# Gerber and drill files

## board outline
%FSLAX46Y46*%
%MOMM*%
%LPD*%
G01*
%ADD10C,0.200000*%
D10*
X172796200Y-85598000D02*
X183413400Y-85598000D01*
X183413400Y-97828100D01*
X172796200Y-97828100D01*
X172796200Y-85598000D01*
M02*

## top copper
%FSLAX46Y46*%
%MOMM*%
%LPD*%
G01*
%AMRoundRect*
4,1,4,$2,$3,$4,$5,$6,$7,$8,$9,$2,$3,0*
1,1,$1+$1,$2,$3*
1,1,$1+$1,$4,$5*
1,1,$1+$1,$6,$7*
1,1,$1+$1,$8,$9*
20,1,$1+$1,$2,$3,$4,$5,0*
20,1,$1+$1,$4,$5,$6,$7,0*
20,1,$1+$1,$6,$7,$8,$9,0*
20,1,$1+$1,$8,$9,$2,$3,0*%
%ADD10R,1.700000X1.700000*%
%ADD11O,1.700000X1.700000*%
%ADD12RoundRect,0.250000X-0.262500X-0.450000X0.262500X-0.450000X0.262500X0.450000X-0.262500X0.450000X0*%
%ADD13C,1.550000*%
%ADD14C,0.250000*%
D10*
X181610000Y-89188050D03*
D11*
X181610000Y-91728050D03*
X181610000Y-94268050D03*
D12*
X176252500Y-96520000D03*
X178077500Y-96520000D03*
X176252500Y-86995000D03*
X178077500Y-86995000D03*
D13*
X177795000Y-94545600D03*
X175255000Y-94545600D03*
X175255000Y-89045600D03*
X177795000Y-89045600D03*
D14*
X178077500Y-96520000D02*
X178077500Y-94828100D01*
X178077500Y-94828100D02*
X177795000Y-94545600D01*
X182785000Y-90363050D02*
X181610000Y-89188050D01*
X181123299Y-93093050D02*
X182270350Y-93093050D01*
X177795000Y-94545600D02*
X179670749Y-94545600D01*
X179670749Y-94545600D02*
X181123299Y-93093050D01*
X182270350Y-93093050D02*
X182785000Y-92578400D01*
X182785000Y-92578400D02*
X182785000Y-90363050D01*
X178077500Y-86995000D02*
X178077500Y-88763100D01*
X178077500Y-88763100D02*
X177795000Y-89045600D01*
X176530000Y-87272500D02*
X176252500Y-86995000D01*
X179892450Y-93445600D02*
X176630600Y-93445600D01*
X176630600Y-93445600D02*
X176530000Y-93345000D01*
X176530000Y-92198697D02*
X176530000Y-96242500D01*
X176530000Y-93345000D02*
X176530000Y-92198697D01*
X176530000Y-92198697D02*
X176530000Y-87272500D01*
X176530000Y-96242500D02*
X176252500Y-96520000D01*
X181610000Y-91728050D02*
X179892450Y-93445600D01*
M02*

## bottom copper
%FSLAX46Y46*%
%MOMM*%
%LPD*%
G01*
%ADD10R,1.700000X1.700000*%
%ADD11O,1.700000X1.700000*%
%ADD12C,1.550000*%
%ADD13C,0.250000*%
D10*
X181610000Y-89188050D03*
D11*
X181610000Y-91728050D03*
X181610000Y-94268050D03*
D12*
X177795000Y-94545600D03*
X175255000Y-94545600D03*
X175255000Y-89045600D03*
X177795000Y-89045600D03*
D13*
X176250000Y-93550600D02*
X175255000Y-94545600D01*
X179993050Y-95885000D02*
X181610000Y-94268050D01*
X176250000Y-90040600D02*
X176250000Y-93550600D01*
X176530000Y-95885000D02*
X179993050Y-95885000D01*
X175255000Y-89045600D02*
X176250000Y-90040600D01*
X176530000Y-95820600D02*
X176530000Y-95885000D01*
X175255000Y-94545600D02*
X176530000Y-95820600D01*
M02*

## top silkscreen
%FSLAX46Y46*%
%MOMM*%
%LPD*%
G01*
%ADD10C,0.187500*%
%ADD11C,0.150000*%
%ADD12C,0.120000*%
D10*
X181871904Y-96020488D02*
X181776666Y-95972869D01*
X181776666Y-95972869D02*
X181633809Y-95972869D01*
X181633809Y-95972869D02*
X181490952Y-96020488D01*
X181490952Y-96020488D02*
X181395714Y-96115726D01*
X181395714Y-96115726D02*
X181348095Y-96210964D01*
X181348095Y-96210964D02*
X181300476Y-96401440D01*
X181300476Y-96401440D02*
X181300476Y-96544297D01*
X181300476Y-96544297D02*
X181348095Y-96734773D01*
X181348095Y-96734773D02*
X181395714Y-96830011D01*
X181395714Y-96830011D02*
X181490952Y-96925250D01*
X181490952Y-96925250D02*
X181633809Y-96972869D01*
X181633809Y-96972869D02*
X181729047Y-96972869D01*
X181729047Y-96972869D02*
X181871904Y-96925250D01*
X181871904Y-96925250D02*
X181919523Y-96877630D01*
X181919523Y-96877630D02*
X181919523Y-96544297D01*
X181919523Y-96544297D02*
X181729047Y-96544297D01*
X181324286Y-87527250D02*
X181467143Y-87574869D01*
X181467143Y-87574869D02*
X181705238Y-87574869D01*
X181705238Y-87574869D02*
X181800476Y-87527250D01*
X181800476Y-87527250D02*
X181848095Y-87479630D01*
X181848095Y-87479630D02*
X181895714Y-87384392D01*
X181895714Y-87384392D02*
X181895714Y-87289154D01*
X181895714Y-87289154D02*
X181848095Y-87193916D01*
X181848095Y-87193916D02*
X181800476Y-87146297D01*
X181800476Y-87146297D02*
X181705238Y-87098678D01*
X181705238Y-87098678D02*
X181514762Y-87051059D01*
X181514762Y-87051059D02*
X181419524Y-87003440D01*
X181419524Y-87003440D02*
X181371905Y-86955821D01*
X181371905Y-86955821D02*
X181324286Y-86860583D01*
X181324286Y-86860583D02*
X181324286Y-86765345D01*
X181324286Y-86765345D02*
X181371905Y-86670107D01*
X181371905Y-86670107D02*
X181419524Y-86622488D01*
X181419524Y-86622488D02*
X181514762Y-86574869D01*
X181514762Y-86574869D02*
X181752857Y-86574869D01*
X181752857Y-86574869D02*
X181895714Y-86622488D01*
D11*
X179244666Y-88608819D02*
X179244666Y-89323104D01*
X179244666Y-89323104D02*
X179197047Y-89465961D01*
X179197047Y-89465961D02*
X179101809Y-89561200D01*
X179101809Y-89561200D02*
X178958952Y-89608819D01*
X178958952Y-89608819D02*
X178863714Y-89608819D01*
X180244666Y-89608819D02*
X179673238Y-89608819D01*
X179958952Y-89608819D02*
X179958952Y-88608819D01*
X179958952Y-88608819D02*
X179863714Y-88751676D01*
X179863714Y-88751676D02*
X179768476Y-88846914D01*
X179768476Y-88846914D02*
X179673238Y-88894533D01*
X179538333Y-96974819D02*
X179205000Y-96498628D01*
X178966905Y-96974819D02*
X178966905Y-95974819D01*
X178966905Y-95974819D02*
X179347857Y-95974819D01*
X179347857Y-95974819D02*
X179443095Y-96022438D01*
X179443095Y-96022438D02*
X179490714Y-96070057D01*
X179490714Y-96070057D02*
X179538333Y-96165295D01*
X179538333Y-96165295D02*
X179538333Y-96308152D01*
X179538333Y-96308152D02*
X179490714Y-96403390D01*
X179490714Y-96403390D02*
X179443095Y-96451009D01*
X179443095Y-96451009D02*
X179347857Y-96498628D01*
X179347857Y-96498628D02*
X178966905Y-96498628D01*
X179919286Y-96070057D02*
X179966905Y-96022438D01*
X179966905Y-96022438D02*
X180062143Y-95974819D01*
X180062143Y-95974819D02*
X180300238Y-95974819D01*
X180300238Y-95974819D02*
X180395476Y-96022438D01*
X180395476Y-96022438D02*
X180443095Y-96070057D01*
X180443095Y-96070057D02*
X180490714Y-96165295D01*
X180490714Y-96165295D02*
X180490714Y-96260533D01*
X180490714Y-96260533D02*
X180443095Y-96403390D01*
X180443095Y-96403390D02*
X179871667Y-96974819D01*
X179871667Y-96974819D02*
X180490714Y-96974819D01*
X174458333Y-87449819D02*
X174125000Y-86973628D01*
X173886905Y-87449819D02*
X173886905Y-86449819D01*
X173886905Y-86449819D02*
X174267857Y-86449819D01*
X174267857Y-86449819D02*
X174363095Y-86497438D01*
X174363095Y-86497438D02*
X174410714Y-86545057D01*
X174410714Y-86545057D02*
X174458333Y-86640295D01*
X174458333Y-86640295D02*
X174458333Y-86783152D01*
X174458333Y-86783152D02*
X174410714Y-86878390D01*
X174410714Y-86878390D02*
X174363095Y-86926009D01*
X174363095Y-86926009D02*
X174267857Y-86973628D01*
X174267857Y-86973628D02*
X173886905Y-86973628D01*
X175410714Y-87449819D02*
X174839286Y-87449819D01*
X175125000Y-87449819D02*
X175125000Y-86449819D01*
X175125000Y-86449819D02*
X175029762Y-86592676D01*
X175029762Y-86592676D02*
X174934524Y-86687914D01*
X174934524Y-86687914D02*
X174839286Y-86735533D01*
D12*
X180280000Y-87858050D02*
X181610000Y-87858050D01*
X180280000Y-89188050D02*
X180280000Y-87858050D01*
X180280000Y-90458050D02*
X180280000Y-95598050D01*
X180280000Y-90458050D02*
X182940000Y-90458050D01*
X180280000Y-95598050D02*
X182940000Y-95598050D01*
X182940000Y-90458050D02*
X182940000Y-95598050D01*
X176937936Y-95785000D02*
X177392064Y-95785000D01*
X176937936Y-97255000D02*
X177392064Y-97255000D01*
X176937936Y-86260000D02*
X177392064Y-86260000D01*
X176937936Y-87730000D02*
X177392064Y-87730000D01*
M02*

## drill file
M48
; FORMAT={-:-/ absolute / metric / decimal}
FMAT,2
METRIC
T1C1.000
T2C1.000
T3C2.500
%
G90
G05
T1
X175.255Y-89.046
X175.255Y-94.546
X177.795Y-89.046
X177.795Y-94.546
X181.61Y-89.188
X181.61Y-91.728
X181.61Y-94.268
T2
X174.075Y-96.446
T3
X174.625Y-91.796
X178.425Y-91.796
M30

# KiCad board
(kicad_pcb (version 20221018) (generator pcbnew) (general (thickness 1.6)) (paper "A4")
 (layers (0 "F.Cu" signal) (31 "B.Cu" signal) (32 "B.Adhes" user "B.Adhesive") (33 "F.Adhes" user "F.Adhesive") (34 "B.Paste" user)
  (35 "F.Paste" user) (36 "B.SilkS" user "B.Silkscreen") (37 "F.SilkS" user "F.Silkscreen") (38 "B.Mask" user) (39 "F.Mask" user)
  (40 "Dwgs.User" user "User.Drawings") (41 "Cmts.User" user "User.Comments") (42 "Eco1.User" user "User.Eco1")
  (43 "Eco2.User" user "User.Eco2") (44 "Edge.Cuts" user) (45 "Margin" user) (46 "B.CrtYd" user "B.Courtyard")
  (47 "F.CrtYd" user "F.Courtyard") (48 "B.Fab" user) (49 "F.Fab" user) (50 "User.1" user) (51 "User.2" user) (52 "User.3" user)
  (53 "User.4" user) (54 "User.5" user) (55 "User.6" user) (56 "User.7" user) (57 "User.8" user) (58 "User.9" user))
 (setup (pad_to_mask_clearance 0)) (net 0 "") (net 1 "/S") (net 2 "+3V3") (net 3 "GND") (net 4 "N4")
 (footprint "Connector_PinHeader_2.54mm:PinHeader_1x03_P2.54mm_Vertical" (layer "F.Cu") (at 181.61 89.18805)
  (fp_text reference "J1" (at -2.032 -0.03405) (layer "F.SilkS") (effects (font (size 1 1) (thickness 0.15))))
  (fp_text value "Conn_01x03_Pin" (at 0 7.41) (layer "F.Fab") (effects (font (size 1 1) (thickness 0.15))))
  (fp_line (start -1.33 -1.33) (end 0 -1.33) (stroke (width 0.12) (type solid)) (layer "F.SilkS"))
  (fp_line (start -1.33 0) (end -1.33 -1.33) (stroke (width 0.12) (type solid)) (layer "F.SilkS"))
  (fp_line (start -1.33 1.27) (end -1.33 6.41) (stroke (width 0.12) (type solid)) (layer "F.SilkS"))
  (fp_line (start -1.33 1.27) (end 1.33 1.27) (stroke (width 0.12) (type solid)) (layer "F.SilkS"))
  (fp_line (start -1.33 6.41) (end 1.33 6.41) (stroke (width 0.12) (type solid)) (layer "F.SilkS"))
  (fp_line (start 1.33 1.27) (end 1.33 6.41) (stroke (width 0.12) (type solid)) (layer "F.SilkS"))
  (pad "1" thru_hole rect (at 0 0) (size 1.7 1.7) (drill 1) (layers "*.Cu" "*.Mask") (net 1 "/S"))
  (pad "2" thru_hole oval (at 0 2.54) (size 1.7 1.7) (drill 1) (layers "*.Cu" "*.Mask") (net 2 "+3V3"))
  (pad "3" thru_hole oval (at 0 5.08) (size 1.7 1.7) (drill 1) (layers "*.Cu" "*.Mask") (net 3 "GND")))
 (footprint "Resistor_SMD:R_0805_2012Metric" (layer "F.Cu") (at 177.165 96.52)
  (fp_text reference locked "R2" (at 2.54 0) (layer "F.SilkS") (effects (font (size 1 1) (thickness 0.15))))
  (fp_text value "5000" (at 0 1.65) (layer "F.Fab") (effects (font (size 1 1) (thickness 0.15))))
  (fp_line (start -0.227064 -0.735) (end 0.227064 -0.735) (stroke (width 0.12) (type solid)) (layer "F.SilkS"))
  (fp_line (start -0.227064 0.735) (end 0.227064 0.735) (stroke (width 0.12) (type solid)) (layer "F.SilkS"))
  (pad "1" smd roundrect (at -0.9125 0) (size 1.025 1.4) (layers "F.Cu" "F.Paste" "F.Mask") (roundrect_rratio 0.243902439) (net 2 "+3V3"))
  (pad "2" smd roundrect (at 0.9125 0) (size 1.025 1.4) (layers "F.Cu" "F.Paste" "F.Mask") (roundrect_rratio 0.243902439) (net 1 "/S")))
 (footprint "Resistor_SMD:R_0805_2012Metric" (layer "F.Cu") (at 177.165 86.995)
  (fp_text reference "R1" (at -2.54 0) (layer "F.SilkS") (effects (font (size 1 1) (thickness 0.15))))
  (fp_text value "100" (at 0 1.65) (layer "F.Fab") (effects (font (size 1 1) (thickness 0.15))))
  (fp_line (start -0.227064 -0.735) (end 0.227064 -0.735) (stroke (width 0.12) (type solid)) (layer "F.SilkS"))
  (fp_line (start -0.227064 0.735) (end 0.227064 0.735) (stroke (width 0.12) (type solid)) (layer "F.SilkS"))
  (pad "1" smd roundrect (at -0.9125 0) (size 1.025 1.4) (layers "F.Cu" "F.Paste" "F.Mask") (roundrect_rratio 0.243902439) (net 2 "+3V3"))
  (pad "2" smd roundrect (at 0.9125 0) (size 1.025 1.4) (layers "F.Cu" "F.Paste" "F.Mask") (roundrect_rratio 0.243902439) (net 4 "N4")))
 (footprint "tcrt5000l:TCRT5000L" (layer "B.Cu") (at 176.525 91.7956 90)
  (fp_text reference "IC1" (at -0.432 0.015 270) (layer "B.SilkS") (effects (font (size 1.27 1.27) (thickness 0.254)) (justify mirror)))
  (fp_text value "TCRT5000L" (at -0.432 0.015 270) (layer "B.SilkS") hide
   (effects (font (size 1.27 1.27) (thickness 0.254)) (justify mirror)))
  (pad "" np_thru_hole circle (at -4.65 -2.45 90) (size 0.001 0.001) (drill 1) (layers "*.Cu" "*.Mask"))
  (pad "" np_thru_hole circle (at 0 -1.9 90) (size 0.001 0.001) (drill 2.5) (layers "*.Cu" "*.Mask"))
  (pad "" np_thru_hole circle (at 0 1.9 90) (size 0.001 0.001) (drill 2.5) (layers "*.Cu" "*.Mask"))
  (pad "1" thru_hole circle (at -2.75 1.27 90) (size 1.55 1.55) (drill 1) (layers "*.Cu" "*.Mask") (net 1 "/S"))
  (pad "2" thru_hole circle (at -2.75 -1.27 90) (size 1.55 1.55) (drill 1) (layers "*.Cu" "*.Mask") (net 3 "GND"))
  (pad "3" thru_hole circle (at 2.75 -1.27 90) (size 1.55 1.55) (drill 1) (layers "*.Cu" "*.Mask") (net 3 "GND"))
  (pad "4" thru_hole circle (at 2.75 1.27 90) (size 1.55 1.55) (drill 1) (layers "*.Cu" "*.Mask") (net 4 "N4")))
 (gr_rect (start 172.7962 85.598) (end 183.4134 97.8281) (stroke (width 0.2) (type solid)) (fill none) (layer "Edge.Cuts"))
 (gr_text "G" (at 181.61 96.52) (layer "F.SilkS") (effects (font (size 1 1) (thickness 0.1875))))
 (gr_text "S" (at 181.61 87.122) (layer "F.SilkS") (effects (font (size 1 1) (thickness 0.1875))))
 (segment (start 178.0775 96.52) (end 178.0775 94.8281) (width 0.25) (layer "F.Cu") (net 1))
 (segment (start 178.0775 94.8281) (end 177.795 94.5456) (width 0.25) (layer "F.Cu") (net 1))
 (segment (start 182.785 90.36305) (end 181.61 89.18805) (width 0.25) (layer "F.Cu") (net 1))
 (segment (start 181.123299 93.09305) (end 182.27035 93.09305) (width 0.25) (layer "F.Cu") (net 1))
 (segment (start 177.795 94.5456) (end 179.670749 94.5456) (width 0.25) (layer "F.Cu") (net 1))
 (segment (start 179.670749 94.5456) (end 181.123299 93.09305) (width 0.25) (layer "F.Cu") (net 1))
 (segment (start 182.27035 93.09305) (end 182.785 92.5784) (width 0.25) (layer "F.Cu") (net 1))
 (segment (start 182.785 92.5784) (end 182.785 90.36305) (width 0.25) (layer "F.Cu") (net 1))
 (segment (start 176.25 93.5506) (end 175.255 94.5456) (width 0.25) (layer "B.Cu") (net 3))
 (segment (start 179.99305 95.885) (end 181.61 94.26805) (width 0.25) (layer "B.Cu") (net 3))
 (segment (start 176.25 90.0406) (end 176.25 93.5506) (width 0.25) (layer "B.Cu") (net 3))
 (segment (start 176.53 95.885) (end 179.99305 95.885) (width 0.25) (layer "B.Cu") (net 3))
 (segment (start 175.255 89.0456) (end 176.25 90.0406) (width 0.25) (layer "B.Cu") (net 3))
 (segment (start 176.53 95.8206) (end 176.53 95.885) (width 0.25) (layer "B.Cu") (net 3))
 (segment (start 175.255 94.5456) (end 176.53 95.8206) (width 0.25) (layer "B.Cu") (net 3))
 (segment (start 178.0775 86.995) (end 178.0775 88.7631) (width 0.25) (layer "F.Cu") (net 4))
 (segment (start 178.0775 88.7631) (end 177.795 89.0456) (width 0.25) (layer "F.Cu") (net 4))
 (segment (start 176.53 87.2725) (end 176.2525 86.995) (width 0.25) (layer "F.Cu") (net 2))
 (segment (start 179.89245 93.4456) (end 176.6306 93.4456) (width 0.25) (layer "F.Cu") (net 2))
 (segment (start 176.6306 93.4456) (end 176.53 93.345) (width 0.25) (layer "F.Cu") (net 2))
 (segment (start 176.53 92.198697) (end 176.53 96.2425) (width 0.25) (layer "F.Cu") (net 2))
 (segment (start 176.53 93.345) (end 176.53 92.198697) (width 0.25) (layer "F.Cu") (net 2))
 (segment (start 176.53 92.198697) (end 176.53 87.2725) (width 0.25) (layer "F.Cu") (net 2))
 (segment (start 176.53 96.2425) (end 176.2525 96.52) (width 0.25) (layer "F.Cu") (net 2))
 (segment (start 181.61 91.72805) (end 179.89245 93.4456) (width 0.25) (layer "F.Cu") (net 2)))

